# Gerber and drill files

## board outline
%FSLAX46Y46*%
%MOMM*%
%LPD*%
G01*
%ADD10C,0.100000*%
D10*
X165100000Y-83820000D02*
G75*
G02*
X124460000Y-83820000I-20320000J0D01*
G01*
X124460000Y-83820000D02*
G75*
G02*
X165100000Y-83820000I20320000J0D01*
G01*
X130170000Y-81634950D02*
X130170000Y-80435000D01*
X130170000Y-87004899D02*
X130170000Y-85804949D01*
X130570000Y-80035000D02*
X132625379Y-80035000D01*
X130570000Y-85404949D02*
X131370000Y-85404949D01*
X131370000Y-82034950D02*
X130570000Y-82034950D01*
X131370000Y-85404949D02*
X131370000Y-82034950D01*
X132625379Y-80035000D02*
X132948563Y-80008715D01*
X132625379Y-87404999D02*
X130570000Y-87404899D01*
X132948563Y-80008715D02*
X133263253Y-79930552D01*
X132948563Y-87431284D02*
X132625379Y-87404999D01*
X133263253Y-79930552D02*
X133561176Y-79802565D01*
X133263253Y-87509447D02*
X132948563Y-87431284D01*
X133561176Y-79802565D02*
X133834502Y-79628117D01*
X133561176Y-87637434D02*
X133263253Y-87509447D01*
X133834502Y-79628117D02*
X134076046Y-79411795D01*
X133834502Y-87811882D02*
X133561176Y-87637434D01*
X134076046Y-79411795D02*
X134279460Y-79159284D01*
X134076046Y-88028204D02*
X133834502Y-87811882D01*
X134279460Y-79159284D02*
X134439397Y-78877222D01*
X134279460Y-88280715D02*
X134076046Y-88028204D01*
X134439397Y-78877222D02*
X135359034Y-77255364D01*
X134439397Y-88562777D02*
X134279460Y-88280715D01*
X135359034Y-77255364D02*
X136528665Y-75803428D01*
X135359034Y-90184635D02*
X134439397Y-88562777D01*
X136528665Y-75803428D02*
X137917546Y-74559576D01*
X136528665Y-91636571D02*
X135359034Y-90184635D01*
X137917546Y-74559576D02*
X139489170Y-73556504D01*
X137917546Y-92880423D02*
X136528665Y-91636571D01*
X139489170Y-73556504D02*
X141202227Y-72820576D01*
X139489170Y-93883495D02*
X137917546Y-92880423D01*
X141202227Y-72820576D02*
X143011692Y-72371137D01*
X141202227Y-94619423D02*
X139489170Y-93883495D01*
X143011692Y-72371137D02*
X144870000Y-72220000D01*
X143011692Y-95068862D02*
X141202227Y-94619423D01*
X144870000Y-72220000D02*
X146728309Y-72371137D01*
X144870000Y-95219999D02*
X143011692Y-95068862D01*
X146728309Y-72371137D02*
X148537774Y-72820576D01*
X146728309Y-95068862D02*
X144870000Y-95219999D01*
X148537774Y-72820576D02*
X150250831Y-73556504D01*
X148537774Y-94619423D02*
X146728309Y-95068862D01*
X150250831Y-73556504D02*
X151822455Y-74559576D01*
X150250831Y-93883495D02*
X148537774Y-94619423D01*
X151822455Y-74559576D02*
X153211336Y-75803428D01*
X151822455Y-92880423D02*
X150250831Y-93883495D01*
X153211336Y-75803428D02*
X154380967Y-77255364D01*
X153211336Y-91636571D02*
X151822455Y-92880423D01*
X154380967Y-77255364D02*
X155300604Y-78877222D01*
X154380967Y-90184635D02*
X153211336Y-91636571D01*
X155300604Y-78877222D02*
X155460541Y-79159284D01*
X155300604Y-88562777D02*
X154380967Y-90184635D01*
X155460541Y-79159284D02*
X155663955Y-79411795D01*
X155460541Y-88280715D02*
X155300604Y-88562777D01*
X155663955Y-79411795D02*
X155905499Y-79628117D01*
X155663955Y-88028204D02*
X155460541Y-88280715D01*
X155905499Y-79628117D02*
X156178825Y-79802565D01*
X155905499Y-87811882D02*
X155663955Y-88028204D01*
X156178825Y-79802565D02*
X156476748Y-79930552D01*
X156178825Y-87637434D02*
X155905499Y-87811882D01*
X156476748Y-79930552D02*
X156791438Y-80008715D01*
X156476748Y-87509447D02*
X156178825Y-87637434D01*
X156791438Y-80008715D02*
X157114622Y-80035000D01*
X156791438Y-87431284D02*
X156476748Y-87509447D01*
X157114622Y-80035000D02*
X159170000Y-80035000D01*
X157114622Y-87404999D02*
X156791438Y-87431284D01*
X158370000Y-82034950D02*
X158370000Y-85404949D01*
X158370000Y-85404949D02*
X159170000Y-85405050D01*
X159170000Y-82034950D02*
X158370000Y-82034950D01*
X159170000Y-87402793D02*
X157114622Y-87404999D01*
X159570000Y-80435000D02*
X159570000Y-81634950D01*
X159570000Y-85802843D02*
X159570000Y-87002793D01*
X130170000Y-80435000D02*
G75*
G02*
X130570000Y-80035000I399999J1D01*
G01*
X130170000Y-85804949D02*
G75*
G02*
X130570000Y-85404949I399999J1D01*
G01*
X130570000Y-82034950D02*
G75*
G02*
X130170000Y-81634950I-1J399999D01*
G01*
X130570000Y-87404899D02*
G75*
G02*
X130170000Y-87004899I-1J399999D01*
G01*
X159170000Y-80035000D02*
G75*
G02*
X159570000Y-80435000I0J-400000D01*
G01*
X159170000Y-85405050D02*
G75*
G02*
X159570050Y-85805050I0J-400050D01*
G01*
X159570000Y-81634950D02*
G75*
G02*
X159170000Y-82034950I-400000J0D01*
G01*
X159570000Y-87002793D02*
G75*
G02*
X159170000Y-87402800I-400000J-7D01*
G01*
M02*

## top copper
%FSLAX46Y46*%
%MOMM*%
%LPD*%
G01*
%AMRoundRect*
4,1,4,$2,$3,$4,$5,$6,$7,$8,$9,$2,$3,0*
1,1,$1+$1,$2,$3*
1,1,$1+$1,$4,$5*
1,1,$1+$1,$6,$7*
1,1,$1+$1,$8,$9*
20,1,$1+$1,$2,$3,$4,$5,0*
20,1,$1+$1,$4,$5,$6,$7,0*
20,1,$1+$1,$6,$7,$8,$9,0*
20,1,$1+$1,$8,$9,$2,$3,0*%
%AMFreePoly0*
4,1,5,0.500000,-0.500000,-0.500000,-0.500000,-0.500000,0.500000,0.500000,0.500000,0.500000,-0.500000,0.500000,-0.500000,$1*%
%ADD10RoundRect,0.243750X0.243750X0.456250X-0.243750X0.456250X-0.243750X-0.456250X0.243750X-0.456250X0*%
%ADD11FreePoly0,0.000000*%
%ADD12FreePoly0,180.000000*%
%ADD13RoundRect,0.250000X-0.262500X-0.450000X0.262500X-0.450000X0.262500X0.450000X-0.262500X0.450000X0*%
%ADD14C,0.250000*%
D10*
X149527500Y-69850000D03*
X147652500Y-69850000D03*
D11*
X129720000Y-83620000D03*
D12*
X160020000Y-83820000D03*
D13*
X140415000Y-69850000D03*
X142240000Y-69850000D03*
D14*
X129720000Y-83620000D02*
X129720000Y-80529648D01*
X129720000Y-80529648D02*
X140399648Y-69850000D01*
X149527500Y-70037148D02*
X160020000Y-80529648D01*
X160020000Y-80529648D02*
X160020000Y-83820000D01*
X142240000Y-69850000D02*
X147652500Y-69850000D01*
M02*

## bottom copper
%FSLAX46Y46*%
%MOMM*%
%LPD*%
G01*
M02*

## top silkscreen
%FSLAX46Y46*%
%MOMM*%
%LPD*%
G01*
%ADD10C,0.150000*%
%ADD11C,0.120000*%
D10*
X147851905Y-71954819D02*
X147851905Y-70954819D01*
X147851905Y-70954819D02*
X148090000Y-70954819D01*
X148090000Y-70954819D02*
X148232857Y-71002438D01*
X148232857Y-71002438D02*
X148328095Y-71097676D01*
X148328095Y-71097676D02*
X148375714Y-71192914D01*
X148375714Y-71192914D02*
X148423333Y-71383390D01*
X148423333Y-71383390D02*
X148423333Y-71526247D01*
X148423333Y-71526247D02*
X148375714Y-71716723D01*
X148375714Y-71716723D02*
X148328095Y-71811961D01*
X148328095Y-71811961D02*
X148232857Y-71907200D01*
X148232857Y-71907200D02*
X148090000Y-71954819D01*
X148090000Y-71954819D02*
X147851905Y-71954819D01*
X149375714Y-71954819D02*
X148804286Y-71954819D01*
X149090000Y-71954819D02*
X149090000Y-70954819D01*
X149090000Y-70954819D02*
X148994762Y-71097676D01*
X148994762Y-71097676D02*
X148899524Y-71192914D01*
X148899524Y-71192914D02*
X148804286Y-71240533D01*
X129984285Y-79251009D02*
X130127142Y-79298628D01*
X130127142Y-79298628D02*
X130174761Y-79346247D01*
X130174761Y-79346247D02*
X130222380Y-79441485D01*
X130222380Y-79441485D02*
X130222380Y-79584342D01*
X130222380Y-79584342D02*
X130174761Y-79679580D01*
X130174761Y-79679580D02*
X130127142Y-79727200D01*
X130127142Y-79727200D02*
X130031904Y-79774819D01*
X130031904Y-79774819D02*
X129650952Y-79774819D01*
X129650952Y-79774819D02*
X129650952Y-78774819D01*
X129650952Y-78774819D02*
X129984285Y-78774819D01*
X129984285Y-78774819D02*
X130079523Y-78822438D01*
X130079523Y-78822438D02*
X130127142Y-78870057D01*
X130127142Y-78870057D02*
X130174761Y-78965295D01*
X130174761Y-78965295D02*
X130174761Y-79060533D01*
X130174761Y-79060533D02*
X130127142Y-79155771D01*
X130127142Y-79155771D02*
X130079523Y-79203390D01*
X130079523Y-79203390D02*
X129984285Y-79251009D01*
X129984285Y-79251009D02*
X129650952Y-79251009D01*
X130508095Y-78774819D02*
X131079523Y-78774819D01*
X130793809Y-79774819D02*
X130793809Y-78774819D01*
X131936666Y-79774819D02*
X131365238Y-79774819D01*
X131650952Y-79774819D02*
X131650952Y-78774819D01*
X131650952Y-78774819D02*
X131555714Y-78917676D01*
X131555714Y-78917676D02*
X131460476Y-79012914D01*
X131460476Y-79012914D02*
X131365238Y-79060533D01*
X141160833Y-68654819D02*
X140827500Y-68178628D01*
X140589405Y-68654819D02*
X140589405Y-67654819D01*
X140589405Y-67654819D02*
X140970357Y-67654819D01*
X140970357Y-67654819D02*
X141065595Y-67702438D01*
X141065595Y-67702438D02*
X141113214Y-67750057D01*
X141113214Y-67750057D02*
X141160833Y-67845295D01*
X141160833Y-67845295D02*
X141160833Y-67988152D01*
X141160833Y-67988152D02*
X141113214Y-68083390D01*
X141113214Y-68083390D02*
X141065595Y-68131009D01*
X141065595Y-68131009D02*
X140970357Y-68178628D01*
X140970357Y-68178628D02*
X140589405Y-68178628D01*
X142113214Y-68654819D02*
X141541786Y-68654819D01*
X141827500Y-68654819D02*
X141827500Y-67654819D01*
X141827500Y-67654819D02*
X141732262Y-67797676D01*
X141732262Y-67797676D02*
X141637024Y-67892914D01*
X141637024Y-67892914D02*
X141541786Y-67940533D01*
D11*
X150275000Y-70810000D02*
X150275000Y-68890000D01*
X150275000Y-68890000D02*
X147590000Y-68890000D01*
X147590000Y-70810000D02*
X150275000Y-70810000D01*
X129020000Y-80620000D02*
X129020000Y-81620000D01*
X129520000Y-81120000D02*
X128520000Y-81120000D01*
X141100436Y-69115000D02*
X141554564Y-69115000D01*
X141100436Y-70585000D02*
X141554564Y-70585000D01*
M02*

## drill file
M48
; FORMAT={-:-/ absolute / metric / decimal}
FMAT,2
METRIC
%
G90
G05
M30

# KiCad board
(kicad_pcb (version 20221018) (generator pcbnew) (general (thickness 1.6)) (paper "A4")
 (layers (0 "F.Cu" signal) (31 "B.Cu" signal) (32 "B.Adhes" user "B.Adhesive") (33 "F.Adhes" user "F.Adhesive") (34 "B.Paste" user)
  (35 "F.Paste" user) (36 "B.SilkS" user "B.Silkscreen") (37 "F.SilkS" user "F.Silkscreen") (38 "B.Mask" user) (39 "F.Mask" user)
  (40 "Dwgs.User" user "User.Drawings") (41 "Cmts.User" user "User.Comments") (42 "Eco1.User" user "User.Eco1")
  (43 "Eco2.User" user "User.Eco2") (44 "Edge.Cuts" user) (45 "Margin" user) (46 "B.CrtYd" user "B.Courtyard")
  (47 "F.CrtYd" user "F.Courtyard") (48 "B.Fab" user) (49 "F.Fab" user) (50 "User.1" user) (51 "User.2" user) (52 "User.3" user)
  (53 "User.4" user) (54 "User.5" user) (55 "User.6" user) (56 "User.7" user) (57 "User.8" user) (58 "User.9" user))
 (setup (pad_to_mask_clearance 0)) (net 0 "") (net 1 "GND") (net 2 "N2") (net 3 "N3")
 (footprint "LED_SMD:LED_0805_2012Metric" (layer "F.Cu") (at 148.59 69.85 180)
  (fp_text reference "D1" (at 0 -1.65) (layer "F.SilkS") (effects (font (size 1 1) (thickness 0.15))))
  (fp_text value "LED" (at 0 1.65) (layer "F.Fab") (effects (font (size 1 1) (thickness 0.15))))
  (fp_line (start -1.685 -0.96) (end -1.685 0.96) (stroke (width 0.12) (type solid)) (layer "F.SilkS"))
  (fp_line (start -1.685 0.96) (end 1 0.96) (stroke (width 0.12) (type solid)) (layer "F.SilkS"))
  (fp_line (start 1 -0.96) (end -1.685 -0.96) (stroke (width 0.12) (type solid)) (layer "F.SilkS"))
  (pad "1" smd roundrect (at -0.9375 0 180) (size 0.975 1.4) (layers "F.Cu" "F.Paste" "F.Mask") (roundrect_rratio 0.25) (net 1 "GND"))
  (pad "2" smd roundrect (at 0.9375 0 180) (size 0.975 1.4) (layers "F.Cu" "F.Paste" "F.Mask") (roundrect_rratio 0.25) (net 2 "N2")))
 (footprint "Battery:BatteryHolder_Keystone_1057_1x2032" (layer "F.Cu") (at 144.87 83.72)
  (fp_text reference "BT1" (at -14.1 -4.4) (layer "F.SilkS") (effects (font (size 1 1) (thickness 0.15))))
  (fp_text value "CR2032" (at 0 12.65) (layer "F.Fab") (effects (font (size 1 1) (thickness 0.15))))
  (fp_line (start -15.85 -3.1) (end -15.85 -2.1) (stroke (width 0.12) (type solid)) (layer "F.SilkS"))
  (fp_line (start -15.35 -2.6) (end -16.35 -2.6) (stroke (width 0.12) (type solid)) (layer "F.SilkS"))
  (fp_line (start -14.7 -2.08505) (end -14.7 -3.285) (stroke (width 0.1) (type solid)) (layer "Edge.Cuts"))
  (fp_line (start -14.7 3.284899) (end -14.7 2.084949) (stroke (width 0.1) (type solid)) (layer "Edge.Cuts"))
  (fp_line (start -14.3 -3.685) (end -12.244621 -3.685) (stroke (width 0.1) (type solid)) (layer "Edge.Cuts"))
  (fp_line (start -14.3 1.684949) (end -13.5 1.684949) (stroke (width 0.1) (type solid)) (layer "Edge.Cuts"))
  (fp_line (start -13.5 -1.68505) (end -14.3 -1.68505) (stroke (width 0.1) (type solid)) (layer "Edge.Cuts"))
  (fp_line (start -13.5 1.684949) (end -13.5 -1.68505) (stroke (width 0.1) (type solid)) (layer "Edge.Cuts"))
  (fp_line (start -12.244621 -3.685) (end -11.921437 -3.711285) (stroke (width 0.1) (type solid)) (layer "Edge.Cuts"))
  (fp_line (start -12.244621 3.684999) (end -14.3 3.684899) (stroke (width 0.1) (type solid)) (layer "Edge.Cuts"))
  (fp_line (start -11.921437 -3.711285) (end -11.606747 -3.789448) (stroke (width 0.1) (type solid)) (layer "Edge.Cuts"))
  (fp_line (start -11.921437 3.711284) (end -12.244621 3.684999) (stroke (width 0.1) (type solid)) (layer "Edge.Cuts"))
  (fp_line (start -11.606747 -3.789448) (end -11.308824 -3.917435) (stroke (width 0.1) (type solid)) (layer "Edge.Cuts"))
  (fp_line (start -11.606747 3.789447) (end -11.921437 3.711284) (stroke (width 0.1) (type solid)) (layer "Edge.Cuts"))
  (fp_line (start -11.308824 -3.917435) (end -11.035498 -4.091883) (stroke (width 0.1) (type solid)) (layer "Edge.Cuts"))
  (fp_line (start -11.308824 3.917434) (end -11.606747 3.789447) (stroke (width 0.1) (type solid)) (layer "Edge.Cuts"))
  (fp_line (start -11.035498 -4.091883) (end -10.793954 -4.308205) (stroke (width 0.1) (type solid)) (layer "Edge.Cuts"))
  (fp_line (start -11.035498 4.091882) (end -11.308824 3.917434) (stroke (width 0.1) (type solid)) (layer "Edge.Cuts"))
  (fp_line (start -10.793954 -4.308205) (end -10.59054 -4.560716) (stroke (width 0.1) (type solid)) (layer "Edge.Cuts"))
  (fp_line (start -10.793954 4.308204) (end -11.035498 4.091882) (stroke (width 0.1) (type solid)) (layer "Edge.Cuts"))
  (fp_line (start -10.59054 -4.560716) (end -10.430603 -4.842778) (stroke (width 0.1) (type solid)) (layer "Edge.Cuts"))
  (fp_line (start -10.59054 4.560715) (end -10.793954 4.308204) (stroke (width 0.1) (type solid)) (layer "Edge.Cuts"))
  (fp_line (start -10.430603 -4.842778) (end -9.510966 -6.464636) (stroke (width 0.1) (type solid)) (layer "Edge.Cuts"))
  (fp_line (start -10.430603 4.842777) (end -10.59054 4.560715) (stroke (width 0.1) (type solid)) (layer "Edge.Cuts"))
  (fp_line (start -9.510966 -6.464636) (end -8.341335 -7.916572) (stroke (width 0.1) (type solid)) (layer "Edge.Cuts"))
  (fp_line (start -9.510966 6.464635) (end -10.430603 4.842777) (stroke (width 0.1) (type solid)) (layer "Edge.Cuts"))
  (fp_line (start -8.341335 -7.916572) (end -6.952454 -9.160424) (stroke (width 0.1) (type solid)) (layer "Edge.Cuts"))
  (fp_line (start -8.341335 7.916571) (end -9.510966 6.464635) (stroke (width 0.1) (type solid)) (layer "Edge.Cuts"))
  (fp_line (start -6.952454 -9.160424) (end -5.38083 -10.163496) (stroke (width 0.1) (type solid)) (layer "Edge.Cuts"))
  (fp_line (start -6.952454 9.160423) (end -8.341335 7.916571) (stroke (width 0.1) (type solid)) (layer "Edge.Cuts"))
  (fp_line (start -5.38083 -10.163496) (end -3.667773 -10.899424) (stroke (width 0.1) (type solid)) (layer "Edge.Cuts"))
  (fp_line (start -5.38083 10.163495) (end -6.952454 9.160423) (stroke (width 0.1) (type solid)) (layer "Edge.Cuts"))
  (fp_line (start -3.667773 -10.899424) (end -1.858308 -11.348863) (stroke (width 0.1) (type solid)) (layer "Edge.Cuts"))
  (fp_line (start -3.667773 10.899423) (end -5.38083 10.163495) (stroke (width 0.1) (type solid)) (layer "Edge.Cuts"))
  (fp_line (start -1.858308 -11.348863) (end 0 -11.5) (stroke (width 0.1) (type solid)) (layer "Edge.Cuts"))
  (fp_line (start -1.858308 11.348862) (end -3.667773 10.899423) (stroke (width 0.1) (type solid)) (layer "Edge.Cuts"))
  (fp_line (start 0 -11.5) (end 1.858309 -11.348863) (stroke (width 0.1) (type solid)) (layer "Edge.Cuts"))
  (fp_line (start 0 11.499999) (end -1.858308 11.348862) (stroke (width 0.1) (type solid)) (layer "Edge.Cuts"))
  (fp_line (start 1.858309 -11.348863) (end 3.667774 -10.899424) (stroke (width 0.1) (type solid)) (layer "Edge.Cuts"))
  (fp_line (start 1.858309 11.348862) (end 0 11.499999) (stroke (width 0.1) (type solid)) (layer "Edge.Cuts"))
  (fp_line (start 3.667774 -10.899424) (end 5.380831 -10.163496) (stroke (width 0.1) (type solid)) (layer "Edge.Cuts"))
  (fp_line (start 3.667774 10.899423) (end 1.858309 11.348862) (stroke (width 0.1) (type solid)) (layer "Edge.Cuts"))
  (fp_line (start 5.380831 -10.163496) (end 6.952455 -9.160424) (stroke (width 0.1) (type solid)) (layer "Edge.Cuts"))
  (fp_line (start 5.380831 10.163495) (end 3.667774 10.899423) (stroke (width 0.1) (type solid)) (layer "Edge.Cuts"))
  (fp_line (start 6.952455 -9.160424) (end 8.341336 -7.916572) (stroke (width 0.1) (type solid)) (layer "Edge.Cuts"))
  (fp_line (start 6.952455 9.160423) (end 5.380831 10.163495) (stroke (width 0.1) (type solid)) (layer "Edge.Cuts"))
  (fp_line (start 8.341336 -7.916572) (end 9.510967 -6.464636) (stroke (width 0.1) (type solid)) (layer "Edge.Cuts"))
  (fp_line (start 8.341336 7.916571) (end 6.952455 9.160423) (stroke (width 0.1) (type solid)) (layer "Edge.Cuts"))
  (fp_line (start 9.510967 -6.464636) (end 10.430604 -4.842778) (stroke (width 0.1) (type solid)) (layer "Edge.Cuts"))
  (fp_line (start 9.510967 6.464635) (end 8.341336 7.916571) (stroke (width 0.1) (type solid)) (layer "Edge.Cuts"))
  (fp_line (start 10.430604 -4.842778) (end 10.590541 -4.560716) (stroke (width 0.1) (type solid)) (layer "Edge.Cuts"))
  (fp_line (start 10.430604 4.842777) (end 9.510967 6.464635) (stroke (width 0.1) (type solid)) (layer "Edge.Cuts"))
  (fp_line (start 10.590541 -4.560716) (end 10.793955 -4.308205) (stroke (width 0.1) (type solid)) (layer "Edge.Cuts"))
  (fp_line (start 10.590541 4.560715) (end 10.430604 4.842777) (stroke (width 0.1) (type solid)) (layer "Edge.Cuts"))
  (fp_line (start 10.793955 -4.308205) (end 11.035499 -4.091883) (stroke (width 0.1) (type solid)) (layer "Edge.Cuts"))
  (fp_line (start 10.793955 4.308204) (end 10.590541 4.560715) (stroke (width 0.1) (type solid)) (layer "Edge.Cuts"))
  (fp_line (start 11.035499 -4.091883) (end 11.308825 -3.917435) (stroke (width 0.1) (type solid)) (layer "Edge.Cuts"))
  (fp_line (start 11.035499 4.091882) (end 10.793955 4.308204) (stroke (width 0.1) (type solid)) (layer "Edge.Cuts"))
  (fp_line (start 11.308825 -3.917435) (end 11.606748 -3.789448) (stroke (width 0.1) (type solid)) (layer "Edge.Cuts"))
  (fp_line (start 11.308825 3.917434) (end 11.035499 4.091882) (stroke (width 0.1) (type solid)) (layer "Edge.Cuts"))
  (fp_line (start 11.606748 -3.789448) (end 11.921438 -3.711285) (stroke (width 0.1) (type solid)) (layer "Edge.Cuts"))
  (fp_line (start 11.606748 3.789447) (end 11.308825 3.917434) (stroke (width 0.1) (type solid)) (layer "Edge.Cuts"))
  (fp_line (start 11.921438 -3.711285) (end 12.244622 -3.685) (stroke (width 0.1) (type solid)) (layer "Edge.Cuts"))
  (fp_line (start 11.921438 3.711284) (end 11.606748 3.789447) (stroke (width 0.1) (type solid)) (layer "Edge.Cuts"))
  (fp_line (start 12.244622 -3.685) (end 14.3 -3.685) (stroke (width 0.1) (type solid)) (layer "Edge.Cuts"))
  (fp_line (start 12.244622 3.684999) (end 11.921438 3.711284) (stroke (width 0.1) (type solid)) (layer "Edge.Cuts"))
  (fp_line (start 13.5 -1.68505) (end 13.5 1.684949) (stroke (width 0.1) (type solid)) (layer "Edge.Cuts"))
  (fp_line (start 13.5 1.684949) (end 14.3 1.68505) (stroke (width 0.1) (type solid)) (layer "Edge.Cuts"))
  (fp_line (start 14.3 -1.68505) (end 13.5 -1.68505) (stroke (width 0.1) (type solid)) (layer "Edge.Cuts"))
  (fp_line (start 14.3 3.682793) (end 12.244622 3.684999) (stroke (width 0.1) (type solid)) (layer "Edge.Cuts"))
  (fp_line (start 14.7 -3.285) (end 14.7 -2.08505) (stroke (width 0.1) (type solid)) (layer "Edge.Cuts"))
  (fp_line (start 14.7 2.082843) (end 14.7 3.282793) (stroke (width 0.1) (type solid)) (layer "Edge.Cuts"))
  (fp_arc (start -14.7 -3.285) (mid -14.582843 -3.567843) (end -14.3 -3.685) (stroke (width 0.1) (type solid)) (layer "Edge.Cuts"))
  (fp_arc (start -14.7 2.084949) (mid -14.582843 1.802106) (end -14.3 1.684949) (stroke (width 0.1) (type solid)) (layer "Edge.Cuts"))
  (fp_arc (start -14.3 -1.68505) (mid -14.582843 -1.802207) (end -14.7 -2.08505) (stroke (width 0.1) (type solid)) (layer "Edge.Cuts"))
  (fp_arc (start -14.3 3.684899) (mid -14.582843 3.567742) (end -14.7 3.284899) (stroke (width 0.1) (type solid)) (layer "Edge.Cuts"))
  (fp_arc (start 14.3 -3.685) (mid 14.582843 -3.567843) (end 14.7 -3.285) (stroke (width 0.1) (type solid)) (layer "Edge.Cuts"))
  (fp_arc (start 14.3 1.68505) (mid 14.582825 1.80221) (end 14.7 2.08505) (stroke (width 0.1) (type solid)) (layer "Edge.Cuts"))
  (fp_arc (start 14.7 -2.08505) (mid 14.582843 -1.802207) (end 14.3 -1.68505) (stroke (width 0.1) (type solid)) (layer "Edge.Cuts"))
  (fp_arc (start 14.7 3.282793) (mid 14.582845 3.56564) (end 14.3 3.682793) (stroke (width 0.1) (type solid)) (layer "Edge.Cuts"))
  (pad "1" smd custom (at -15.15 -0.1) (size 1 1) (layers "F.Cu" "F.Paste" "F.Mask") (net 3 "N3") (thermal_bridge_angle 45)
   (options (clearance outline) (anchor rect)) (primitives))
  (pad "2" smd custom (at 15.15 0.1 180) (size 1 1) (layers "F.Cu" "F.Paste" "F.Mask") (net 1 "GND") (thermal_bridge_angle 45)
   (options (clearance outline) (anchor rect)) (primitives)))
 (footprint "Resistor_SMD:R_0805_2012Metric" (layer "F.Cu") (at 141.3275 69.85)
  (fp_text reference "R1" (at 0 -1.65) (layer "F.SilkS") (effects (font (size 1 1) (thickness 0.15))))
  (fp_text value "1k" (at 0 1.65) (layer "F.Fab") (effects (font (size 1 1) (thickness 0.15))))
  (fp_line (start -0.227064 -0.735) (end 0.227064 -0.735) (stroke (width 0.12) (type solid)) (layer "F.SilkS"))
  (fp_line (start -0.227064 0.735) (end 0.227064 0.735) (stroke (width 0.12) (type solid)) (layer "F.SilkS"))
  (pad "1" smd roundrect (at -0.9125 0) (size 1.025 1.4) (layers "F.Cu" "F.Paste" "F.Mask") (roundrect_rratio 0.243902) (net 3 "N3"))
  (pad "2" smd roundrect (at 0.9125 0) (size 1.025 1.4) (layers "F.Cu" "F.Paste" "F.Mask") (roundrect_rratio 0.243902) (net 2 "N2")))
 (gr_circle (center 144.78 83.82) (end 124.46 83.82) (stroke (width 0.1) (type default)) (fill none) (layer "Edge.Cuts"))
 (segment (start 129.72 83.62) (end 129.72 80.529648) (width 0.25) (layer "F.Cu") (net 3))
 (segment (start 129.72 80.529648) (end 140.399648 69.85) (width 0.25) (layer "F.Cu") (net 3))
 (segment (start 149.5275 70.037148) (end 160.02 80.529648) (width 0.25) (layer "F.Cu") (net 1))
 (segment (start 160.02 80.529648) (end 160.02 83.82) (width 0.25) (layer "F.Cu") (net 1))
 (segment (start 142.24 69.85) (end 147.6525 69.85) (width 0.25) (layer "F.Cu") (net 2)))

